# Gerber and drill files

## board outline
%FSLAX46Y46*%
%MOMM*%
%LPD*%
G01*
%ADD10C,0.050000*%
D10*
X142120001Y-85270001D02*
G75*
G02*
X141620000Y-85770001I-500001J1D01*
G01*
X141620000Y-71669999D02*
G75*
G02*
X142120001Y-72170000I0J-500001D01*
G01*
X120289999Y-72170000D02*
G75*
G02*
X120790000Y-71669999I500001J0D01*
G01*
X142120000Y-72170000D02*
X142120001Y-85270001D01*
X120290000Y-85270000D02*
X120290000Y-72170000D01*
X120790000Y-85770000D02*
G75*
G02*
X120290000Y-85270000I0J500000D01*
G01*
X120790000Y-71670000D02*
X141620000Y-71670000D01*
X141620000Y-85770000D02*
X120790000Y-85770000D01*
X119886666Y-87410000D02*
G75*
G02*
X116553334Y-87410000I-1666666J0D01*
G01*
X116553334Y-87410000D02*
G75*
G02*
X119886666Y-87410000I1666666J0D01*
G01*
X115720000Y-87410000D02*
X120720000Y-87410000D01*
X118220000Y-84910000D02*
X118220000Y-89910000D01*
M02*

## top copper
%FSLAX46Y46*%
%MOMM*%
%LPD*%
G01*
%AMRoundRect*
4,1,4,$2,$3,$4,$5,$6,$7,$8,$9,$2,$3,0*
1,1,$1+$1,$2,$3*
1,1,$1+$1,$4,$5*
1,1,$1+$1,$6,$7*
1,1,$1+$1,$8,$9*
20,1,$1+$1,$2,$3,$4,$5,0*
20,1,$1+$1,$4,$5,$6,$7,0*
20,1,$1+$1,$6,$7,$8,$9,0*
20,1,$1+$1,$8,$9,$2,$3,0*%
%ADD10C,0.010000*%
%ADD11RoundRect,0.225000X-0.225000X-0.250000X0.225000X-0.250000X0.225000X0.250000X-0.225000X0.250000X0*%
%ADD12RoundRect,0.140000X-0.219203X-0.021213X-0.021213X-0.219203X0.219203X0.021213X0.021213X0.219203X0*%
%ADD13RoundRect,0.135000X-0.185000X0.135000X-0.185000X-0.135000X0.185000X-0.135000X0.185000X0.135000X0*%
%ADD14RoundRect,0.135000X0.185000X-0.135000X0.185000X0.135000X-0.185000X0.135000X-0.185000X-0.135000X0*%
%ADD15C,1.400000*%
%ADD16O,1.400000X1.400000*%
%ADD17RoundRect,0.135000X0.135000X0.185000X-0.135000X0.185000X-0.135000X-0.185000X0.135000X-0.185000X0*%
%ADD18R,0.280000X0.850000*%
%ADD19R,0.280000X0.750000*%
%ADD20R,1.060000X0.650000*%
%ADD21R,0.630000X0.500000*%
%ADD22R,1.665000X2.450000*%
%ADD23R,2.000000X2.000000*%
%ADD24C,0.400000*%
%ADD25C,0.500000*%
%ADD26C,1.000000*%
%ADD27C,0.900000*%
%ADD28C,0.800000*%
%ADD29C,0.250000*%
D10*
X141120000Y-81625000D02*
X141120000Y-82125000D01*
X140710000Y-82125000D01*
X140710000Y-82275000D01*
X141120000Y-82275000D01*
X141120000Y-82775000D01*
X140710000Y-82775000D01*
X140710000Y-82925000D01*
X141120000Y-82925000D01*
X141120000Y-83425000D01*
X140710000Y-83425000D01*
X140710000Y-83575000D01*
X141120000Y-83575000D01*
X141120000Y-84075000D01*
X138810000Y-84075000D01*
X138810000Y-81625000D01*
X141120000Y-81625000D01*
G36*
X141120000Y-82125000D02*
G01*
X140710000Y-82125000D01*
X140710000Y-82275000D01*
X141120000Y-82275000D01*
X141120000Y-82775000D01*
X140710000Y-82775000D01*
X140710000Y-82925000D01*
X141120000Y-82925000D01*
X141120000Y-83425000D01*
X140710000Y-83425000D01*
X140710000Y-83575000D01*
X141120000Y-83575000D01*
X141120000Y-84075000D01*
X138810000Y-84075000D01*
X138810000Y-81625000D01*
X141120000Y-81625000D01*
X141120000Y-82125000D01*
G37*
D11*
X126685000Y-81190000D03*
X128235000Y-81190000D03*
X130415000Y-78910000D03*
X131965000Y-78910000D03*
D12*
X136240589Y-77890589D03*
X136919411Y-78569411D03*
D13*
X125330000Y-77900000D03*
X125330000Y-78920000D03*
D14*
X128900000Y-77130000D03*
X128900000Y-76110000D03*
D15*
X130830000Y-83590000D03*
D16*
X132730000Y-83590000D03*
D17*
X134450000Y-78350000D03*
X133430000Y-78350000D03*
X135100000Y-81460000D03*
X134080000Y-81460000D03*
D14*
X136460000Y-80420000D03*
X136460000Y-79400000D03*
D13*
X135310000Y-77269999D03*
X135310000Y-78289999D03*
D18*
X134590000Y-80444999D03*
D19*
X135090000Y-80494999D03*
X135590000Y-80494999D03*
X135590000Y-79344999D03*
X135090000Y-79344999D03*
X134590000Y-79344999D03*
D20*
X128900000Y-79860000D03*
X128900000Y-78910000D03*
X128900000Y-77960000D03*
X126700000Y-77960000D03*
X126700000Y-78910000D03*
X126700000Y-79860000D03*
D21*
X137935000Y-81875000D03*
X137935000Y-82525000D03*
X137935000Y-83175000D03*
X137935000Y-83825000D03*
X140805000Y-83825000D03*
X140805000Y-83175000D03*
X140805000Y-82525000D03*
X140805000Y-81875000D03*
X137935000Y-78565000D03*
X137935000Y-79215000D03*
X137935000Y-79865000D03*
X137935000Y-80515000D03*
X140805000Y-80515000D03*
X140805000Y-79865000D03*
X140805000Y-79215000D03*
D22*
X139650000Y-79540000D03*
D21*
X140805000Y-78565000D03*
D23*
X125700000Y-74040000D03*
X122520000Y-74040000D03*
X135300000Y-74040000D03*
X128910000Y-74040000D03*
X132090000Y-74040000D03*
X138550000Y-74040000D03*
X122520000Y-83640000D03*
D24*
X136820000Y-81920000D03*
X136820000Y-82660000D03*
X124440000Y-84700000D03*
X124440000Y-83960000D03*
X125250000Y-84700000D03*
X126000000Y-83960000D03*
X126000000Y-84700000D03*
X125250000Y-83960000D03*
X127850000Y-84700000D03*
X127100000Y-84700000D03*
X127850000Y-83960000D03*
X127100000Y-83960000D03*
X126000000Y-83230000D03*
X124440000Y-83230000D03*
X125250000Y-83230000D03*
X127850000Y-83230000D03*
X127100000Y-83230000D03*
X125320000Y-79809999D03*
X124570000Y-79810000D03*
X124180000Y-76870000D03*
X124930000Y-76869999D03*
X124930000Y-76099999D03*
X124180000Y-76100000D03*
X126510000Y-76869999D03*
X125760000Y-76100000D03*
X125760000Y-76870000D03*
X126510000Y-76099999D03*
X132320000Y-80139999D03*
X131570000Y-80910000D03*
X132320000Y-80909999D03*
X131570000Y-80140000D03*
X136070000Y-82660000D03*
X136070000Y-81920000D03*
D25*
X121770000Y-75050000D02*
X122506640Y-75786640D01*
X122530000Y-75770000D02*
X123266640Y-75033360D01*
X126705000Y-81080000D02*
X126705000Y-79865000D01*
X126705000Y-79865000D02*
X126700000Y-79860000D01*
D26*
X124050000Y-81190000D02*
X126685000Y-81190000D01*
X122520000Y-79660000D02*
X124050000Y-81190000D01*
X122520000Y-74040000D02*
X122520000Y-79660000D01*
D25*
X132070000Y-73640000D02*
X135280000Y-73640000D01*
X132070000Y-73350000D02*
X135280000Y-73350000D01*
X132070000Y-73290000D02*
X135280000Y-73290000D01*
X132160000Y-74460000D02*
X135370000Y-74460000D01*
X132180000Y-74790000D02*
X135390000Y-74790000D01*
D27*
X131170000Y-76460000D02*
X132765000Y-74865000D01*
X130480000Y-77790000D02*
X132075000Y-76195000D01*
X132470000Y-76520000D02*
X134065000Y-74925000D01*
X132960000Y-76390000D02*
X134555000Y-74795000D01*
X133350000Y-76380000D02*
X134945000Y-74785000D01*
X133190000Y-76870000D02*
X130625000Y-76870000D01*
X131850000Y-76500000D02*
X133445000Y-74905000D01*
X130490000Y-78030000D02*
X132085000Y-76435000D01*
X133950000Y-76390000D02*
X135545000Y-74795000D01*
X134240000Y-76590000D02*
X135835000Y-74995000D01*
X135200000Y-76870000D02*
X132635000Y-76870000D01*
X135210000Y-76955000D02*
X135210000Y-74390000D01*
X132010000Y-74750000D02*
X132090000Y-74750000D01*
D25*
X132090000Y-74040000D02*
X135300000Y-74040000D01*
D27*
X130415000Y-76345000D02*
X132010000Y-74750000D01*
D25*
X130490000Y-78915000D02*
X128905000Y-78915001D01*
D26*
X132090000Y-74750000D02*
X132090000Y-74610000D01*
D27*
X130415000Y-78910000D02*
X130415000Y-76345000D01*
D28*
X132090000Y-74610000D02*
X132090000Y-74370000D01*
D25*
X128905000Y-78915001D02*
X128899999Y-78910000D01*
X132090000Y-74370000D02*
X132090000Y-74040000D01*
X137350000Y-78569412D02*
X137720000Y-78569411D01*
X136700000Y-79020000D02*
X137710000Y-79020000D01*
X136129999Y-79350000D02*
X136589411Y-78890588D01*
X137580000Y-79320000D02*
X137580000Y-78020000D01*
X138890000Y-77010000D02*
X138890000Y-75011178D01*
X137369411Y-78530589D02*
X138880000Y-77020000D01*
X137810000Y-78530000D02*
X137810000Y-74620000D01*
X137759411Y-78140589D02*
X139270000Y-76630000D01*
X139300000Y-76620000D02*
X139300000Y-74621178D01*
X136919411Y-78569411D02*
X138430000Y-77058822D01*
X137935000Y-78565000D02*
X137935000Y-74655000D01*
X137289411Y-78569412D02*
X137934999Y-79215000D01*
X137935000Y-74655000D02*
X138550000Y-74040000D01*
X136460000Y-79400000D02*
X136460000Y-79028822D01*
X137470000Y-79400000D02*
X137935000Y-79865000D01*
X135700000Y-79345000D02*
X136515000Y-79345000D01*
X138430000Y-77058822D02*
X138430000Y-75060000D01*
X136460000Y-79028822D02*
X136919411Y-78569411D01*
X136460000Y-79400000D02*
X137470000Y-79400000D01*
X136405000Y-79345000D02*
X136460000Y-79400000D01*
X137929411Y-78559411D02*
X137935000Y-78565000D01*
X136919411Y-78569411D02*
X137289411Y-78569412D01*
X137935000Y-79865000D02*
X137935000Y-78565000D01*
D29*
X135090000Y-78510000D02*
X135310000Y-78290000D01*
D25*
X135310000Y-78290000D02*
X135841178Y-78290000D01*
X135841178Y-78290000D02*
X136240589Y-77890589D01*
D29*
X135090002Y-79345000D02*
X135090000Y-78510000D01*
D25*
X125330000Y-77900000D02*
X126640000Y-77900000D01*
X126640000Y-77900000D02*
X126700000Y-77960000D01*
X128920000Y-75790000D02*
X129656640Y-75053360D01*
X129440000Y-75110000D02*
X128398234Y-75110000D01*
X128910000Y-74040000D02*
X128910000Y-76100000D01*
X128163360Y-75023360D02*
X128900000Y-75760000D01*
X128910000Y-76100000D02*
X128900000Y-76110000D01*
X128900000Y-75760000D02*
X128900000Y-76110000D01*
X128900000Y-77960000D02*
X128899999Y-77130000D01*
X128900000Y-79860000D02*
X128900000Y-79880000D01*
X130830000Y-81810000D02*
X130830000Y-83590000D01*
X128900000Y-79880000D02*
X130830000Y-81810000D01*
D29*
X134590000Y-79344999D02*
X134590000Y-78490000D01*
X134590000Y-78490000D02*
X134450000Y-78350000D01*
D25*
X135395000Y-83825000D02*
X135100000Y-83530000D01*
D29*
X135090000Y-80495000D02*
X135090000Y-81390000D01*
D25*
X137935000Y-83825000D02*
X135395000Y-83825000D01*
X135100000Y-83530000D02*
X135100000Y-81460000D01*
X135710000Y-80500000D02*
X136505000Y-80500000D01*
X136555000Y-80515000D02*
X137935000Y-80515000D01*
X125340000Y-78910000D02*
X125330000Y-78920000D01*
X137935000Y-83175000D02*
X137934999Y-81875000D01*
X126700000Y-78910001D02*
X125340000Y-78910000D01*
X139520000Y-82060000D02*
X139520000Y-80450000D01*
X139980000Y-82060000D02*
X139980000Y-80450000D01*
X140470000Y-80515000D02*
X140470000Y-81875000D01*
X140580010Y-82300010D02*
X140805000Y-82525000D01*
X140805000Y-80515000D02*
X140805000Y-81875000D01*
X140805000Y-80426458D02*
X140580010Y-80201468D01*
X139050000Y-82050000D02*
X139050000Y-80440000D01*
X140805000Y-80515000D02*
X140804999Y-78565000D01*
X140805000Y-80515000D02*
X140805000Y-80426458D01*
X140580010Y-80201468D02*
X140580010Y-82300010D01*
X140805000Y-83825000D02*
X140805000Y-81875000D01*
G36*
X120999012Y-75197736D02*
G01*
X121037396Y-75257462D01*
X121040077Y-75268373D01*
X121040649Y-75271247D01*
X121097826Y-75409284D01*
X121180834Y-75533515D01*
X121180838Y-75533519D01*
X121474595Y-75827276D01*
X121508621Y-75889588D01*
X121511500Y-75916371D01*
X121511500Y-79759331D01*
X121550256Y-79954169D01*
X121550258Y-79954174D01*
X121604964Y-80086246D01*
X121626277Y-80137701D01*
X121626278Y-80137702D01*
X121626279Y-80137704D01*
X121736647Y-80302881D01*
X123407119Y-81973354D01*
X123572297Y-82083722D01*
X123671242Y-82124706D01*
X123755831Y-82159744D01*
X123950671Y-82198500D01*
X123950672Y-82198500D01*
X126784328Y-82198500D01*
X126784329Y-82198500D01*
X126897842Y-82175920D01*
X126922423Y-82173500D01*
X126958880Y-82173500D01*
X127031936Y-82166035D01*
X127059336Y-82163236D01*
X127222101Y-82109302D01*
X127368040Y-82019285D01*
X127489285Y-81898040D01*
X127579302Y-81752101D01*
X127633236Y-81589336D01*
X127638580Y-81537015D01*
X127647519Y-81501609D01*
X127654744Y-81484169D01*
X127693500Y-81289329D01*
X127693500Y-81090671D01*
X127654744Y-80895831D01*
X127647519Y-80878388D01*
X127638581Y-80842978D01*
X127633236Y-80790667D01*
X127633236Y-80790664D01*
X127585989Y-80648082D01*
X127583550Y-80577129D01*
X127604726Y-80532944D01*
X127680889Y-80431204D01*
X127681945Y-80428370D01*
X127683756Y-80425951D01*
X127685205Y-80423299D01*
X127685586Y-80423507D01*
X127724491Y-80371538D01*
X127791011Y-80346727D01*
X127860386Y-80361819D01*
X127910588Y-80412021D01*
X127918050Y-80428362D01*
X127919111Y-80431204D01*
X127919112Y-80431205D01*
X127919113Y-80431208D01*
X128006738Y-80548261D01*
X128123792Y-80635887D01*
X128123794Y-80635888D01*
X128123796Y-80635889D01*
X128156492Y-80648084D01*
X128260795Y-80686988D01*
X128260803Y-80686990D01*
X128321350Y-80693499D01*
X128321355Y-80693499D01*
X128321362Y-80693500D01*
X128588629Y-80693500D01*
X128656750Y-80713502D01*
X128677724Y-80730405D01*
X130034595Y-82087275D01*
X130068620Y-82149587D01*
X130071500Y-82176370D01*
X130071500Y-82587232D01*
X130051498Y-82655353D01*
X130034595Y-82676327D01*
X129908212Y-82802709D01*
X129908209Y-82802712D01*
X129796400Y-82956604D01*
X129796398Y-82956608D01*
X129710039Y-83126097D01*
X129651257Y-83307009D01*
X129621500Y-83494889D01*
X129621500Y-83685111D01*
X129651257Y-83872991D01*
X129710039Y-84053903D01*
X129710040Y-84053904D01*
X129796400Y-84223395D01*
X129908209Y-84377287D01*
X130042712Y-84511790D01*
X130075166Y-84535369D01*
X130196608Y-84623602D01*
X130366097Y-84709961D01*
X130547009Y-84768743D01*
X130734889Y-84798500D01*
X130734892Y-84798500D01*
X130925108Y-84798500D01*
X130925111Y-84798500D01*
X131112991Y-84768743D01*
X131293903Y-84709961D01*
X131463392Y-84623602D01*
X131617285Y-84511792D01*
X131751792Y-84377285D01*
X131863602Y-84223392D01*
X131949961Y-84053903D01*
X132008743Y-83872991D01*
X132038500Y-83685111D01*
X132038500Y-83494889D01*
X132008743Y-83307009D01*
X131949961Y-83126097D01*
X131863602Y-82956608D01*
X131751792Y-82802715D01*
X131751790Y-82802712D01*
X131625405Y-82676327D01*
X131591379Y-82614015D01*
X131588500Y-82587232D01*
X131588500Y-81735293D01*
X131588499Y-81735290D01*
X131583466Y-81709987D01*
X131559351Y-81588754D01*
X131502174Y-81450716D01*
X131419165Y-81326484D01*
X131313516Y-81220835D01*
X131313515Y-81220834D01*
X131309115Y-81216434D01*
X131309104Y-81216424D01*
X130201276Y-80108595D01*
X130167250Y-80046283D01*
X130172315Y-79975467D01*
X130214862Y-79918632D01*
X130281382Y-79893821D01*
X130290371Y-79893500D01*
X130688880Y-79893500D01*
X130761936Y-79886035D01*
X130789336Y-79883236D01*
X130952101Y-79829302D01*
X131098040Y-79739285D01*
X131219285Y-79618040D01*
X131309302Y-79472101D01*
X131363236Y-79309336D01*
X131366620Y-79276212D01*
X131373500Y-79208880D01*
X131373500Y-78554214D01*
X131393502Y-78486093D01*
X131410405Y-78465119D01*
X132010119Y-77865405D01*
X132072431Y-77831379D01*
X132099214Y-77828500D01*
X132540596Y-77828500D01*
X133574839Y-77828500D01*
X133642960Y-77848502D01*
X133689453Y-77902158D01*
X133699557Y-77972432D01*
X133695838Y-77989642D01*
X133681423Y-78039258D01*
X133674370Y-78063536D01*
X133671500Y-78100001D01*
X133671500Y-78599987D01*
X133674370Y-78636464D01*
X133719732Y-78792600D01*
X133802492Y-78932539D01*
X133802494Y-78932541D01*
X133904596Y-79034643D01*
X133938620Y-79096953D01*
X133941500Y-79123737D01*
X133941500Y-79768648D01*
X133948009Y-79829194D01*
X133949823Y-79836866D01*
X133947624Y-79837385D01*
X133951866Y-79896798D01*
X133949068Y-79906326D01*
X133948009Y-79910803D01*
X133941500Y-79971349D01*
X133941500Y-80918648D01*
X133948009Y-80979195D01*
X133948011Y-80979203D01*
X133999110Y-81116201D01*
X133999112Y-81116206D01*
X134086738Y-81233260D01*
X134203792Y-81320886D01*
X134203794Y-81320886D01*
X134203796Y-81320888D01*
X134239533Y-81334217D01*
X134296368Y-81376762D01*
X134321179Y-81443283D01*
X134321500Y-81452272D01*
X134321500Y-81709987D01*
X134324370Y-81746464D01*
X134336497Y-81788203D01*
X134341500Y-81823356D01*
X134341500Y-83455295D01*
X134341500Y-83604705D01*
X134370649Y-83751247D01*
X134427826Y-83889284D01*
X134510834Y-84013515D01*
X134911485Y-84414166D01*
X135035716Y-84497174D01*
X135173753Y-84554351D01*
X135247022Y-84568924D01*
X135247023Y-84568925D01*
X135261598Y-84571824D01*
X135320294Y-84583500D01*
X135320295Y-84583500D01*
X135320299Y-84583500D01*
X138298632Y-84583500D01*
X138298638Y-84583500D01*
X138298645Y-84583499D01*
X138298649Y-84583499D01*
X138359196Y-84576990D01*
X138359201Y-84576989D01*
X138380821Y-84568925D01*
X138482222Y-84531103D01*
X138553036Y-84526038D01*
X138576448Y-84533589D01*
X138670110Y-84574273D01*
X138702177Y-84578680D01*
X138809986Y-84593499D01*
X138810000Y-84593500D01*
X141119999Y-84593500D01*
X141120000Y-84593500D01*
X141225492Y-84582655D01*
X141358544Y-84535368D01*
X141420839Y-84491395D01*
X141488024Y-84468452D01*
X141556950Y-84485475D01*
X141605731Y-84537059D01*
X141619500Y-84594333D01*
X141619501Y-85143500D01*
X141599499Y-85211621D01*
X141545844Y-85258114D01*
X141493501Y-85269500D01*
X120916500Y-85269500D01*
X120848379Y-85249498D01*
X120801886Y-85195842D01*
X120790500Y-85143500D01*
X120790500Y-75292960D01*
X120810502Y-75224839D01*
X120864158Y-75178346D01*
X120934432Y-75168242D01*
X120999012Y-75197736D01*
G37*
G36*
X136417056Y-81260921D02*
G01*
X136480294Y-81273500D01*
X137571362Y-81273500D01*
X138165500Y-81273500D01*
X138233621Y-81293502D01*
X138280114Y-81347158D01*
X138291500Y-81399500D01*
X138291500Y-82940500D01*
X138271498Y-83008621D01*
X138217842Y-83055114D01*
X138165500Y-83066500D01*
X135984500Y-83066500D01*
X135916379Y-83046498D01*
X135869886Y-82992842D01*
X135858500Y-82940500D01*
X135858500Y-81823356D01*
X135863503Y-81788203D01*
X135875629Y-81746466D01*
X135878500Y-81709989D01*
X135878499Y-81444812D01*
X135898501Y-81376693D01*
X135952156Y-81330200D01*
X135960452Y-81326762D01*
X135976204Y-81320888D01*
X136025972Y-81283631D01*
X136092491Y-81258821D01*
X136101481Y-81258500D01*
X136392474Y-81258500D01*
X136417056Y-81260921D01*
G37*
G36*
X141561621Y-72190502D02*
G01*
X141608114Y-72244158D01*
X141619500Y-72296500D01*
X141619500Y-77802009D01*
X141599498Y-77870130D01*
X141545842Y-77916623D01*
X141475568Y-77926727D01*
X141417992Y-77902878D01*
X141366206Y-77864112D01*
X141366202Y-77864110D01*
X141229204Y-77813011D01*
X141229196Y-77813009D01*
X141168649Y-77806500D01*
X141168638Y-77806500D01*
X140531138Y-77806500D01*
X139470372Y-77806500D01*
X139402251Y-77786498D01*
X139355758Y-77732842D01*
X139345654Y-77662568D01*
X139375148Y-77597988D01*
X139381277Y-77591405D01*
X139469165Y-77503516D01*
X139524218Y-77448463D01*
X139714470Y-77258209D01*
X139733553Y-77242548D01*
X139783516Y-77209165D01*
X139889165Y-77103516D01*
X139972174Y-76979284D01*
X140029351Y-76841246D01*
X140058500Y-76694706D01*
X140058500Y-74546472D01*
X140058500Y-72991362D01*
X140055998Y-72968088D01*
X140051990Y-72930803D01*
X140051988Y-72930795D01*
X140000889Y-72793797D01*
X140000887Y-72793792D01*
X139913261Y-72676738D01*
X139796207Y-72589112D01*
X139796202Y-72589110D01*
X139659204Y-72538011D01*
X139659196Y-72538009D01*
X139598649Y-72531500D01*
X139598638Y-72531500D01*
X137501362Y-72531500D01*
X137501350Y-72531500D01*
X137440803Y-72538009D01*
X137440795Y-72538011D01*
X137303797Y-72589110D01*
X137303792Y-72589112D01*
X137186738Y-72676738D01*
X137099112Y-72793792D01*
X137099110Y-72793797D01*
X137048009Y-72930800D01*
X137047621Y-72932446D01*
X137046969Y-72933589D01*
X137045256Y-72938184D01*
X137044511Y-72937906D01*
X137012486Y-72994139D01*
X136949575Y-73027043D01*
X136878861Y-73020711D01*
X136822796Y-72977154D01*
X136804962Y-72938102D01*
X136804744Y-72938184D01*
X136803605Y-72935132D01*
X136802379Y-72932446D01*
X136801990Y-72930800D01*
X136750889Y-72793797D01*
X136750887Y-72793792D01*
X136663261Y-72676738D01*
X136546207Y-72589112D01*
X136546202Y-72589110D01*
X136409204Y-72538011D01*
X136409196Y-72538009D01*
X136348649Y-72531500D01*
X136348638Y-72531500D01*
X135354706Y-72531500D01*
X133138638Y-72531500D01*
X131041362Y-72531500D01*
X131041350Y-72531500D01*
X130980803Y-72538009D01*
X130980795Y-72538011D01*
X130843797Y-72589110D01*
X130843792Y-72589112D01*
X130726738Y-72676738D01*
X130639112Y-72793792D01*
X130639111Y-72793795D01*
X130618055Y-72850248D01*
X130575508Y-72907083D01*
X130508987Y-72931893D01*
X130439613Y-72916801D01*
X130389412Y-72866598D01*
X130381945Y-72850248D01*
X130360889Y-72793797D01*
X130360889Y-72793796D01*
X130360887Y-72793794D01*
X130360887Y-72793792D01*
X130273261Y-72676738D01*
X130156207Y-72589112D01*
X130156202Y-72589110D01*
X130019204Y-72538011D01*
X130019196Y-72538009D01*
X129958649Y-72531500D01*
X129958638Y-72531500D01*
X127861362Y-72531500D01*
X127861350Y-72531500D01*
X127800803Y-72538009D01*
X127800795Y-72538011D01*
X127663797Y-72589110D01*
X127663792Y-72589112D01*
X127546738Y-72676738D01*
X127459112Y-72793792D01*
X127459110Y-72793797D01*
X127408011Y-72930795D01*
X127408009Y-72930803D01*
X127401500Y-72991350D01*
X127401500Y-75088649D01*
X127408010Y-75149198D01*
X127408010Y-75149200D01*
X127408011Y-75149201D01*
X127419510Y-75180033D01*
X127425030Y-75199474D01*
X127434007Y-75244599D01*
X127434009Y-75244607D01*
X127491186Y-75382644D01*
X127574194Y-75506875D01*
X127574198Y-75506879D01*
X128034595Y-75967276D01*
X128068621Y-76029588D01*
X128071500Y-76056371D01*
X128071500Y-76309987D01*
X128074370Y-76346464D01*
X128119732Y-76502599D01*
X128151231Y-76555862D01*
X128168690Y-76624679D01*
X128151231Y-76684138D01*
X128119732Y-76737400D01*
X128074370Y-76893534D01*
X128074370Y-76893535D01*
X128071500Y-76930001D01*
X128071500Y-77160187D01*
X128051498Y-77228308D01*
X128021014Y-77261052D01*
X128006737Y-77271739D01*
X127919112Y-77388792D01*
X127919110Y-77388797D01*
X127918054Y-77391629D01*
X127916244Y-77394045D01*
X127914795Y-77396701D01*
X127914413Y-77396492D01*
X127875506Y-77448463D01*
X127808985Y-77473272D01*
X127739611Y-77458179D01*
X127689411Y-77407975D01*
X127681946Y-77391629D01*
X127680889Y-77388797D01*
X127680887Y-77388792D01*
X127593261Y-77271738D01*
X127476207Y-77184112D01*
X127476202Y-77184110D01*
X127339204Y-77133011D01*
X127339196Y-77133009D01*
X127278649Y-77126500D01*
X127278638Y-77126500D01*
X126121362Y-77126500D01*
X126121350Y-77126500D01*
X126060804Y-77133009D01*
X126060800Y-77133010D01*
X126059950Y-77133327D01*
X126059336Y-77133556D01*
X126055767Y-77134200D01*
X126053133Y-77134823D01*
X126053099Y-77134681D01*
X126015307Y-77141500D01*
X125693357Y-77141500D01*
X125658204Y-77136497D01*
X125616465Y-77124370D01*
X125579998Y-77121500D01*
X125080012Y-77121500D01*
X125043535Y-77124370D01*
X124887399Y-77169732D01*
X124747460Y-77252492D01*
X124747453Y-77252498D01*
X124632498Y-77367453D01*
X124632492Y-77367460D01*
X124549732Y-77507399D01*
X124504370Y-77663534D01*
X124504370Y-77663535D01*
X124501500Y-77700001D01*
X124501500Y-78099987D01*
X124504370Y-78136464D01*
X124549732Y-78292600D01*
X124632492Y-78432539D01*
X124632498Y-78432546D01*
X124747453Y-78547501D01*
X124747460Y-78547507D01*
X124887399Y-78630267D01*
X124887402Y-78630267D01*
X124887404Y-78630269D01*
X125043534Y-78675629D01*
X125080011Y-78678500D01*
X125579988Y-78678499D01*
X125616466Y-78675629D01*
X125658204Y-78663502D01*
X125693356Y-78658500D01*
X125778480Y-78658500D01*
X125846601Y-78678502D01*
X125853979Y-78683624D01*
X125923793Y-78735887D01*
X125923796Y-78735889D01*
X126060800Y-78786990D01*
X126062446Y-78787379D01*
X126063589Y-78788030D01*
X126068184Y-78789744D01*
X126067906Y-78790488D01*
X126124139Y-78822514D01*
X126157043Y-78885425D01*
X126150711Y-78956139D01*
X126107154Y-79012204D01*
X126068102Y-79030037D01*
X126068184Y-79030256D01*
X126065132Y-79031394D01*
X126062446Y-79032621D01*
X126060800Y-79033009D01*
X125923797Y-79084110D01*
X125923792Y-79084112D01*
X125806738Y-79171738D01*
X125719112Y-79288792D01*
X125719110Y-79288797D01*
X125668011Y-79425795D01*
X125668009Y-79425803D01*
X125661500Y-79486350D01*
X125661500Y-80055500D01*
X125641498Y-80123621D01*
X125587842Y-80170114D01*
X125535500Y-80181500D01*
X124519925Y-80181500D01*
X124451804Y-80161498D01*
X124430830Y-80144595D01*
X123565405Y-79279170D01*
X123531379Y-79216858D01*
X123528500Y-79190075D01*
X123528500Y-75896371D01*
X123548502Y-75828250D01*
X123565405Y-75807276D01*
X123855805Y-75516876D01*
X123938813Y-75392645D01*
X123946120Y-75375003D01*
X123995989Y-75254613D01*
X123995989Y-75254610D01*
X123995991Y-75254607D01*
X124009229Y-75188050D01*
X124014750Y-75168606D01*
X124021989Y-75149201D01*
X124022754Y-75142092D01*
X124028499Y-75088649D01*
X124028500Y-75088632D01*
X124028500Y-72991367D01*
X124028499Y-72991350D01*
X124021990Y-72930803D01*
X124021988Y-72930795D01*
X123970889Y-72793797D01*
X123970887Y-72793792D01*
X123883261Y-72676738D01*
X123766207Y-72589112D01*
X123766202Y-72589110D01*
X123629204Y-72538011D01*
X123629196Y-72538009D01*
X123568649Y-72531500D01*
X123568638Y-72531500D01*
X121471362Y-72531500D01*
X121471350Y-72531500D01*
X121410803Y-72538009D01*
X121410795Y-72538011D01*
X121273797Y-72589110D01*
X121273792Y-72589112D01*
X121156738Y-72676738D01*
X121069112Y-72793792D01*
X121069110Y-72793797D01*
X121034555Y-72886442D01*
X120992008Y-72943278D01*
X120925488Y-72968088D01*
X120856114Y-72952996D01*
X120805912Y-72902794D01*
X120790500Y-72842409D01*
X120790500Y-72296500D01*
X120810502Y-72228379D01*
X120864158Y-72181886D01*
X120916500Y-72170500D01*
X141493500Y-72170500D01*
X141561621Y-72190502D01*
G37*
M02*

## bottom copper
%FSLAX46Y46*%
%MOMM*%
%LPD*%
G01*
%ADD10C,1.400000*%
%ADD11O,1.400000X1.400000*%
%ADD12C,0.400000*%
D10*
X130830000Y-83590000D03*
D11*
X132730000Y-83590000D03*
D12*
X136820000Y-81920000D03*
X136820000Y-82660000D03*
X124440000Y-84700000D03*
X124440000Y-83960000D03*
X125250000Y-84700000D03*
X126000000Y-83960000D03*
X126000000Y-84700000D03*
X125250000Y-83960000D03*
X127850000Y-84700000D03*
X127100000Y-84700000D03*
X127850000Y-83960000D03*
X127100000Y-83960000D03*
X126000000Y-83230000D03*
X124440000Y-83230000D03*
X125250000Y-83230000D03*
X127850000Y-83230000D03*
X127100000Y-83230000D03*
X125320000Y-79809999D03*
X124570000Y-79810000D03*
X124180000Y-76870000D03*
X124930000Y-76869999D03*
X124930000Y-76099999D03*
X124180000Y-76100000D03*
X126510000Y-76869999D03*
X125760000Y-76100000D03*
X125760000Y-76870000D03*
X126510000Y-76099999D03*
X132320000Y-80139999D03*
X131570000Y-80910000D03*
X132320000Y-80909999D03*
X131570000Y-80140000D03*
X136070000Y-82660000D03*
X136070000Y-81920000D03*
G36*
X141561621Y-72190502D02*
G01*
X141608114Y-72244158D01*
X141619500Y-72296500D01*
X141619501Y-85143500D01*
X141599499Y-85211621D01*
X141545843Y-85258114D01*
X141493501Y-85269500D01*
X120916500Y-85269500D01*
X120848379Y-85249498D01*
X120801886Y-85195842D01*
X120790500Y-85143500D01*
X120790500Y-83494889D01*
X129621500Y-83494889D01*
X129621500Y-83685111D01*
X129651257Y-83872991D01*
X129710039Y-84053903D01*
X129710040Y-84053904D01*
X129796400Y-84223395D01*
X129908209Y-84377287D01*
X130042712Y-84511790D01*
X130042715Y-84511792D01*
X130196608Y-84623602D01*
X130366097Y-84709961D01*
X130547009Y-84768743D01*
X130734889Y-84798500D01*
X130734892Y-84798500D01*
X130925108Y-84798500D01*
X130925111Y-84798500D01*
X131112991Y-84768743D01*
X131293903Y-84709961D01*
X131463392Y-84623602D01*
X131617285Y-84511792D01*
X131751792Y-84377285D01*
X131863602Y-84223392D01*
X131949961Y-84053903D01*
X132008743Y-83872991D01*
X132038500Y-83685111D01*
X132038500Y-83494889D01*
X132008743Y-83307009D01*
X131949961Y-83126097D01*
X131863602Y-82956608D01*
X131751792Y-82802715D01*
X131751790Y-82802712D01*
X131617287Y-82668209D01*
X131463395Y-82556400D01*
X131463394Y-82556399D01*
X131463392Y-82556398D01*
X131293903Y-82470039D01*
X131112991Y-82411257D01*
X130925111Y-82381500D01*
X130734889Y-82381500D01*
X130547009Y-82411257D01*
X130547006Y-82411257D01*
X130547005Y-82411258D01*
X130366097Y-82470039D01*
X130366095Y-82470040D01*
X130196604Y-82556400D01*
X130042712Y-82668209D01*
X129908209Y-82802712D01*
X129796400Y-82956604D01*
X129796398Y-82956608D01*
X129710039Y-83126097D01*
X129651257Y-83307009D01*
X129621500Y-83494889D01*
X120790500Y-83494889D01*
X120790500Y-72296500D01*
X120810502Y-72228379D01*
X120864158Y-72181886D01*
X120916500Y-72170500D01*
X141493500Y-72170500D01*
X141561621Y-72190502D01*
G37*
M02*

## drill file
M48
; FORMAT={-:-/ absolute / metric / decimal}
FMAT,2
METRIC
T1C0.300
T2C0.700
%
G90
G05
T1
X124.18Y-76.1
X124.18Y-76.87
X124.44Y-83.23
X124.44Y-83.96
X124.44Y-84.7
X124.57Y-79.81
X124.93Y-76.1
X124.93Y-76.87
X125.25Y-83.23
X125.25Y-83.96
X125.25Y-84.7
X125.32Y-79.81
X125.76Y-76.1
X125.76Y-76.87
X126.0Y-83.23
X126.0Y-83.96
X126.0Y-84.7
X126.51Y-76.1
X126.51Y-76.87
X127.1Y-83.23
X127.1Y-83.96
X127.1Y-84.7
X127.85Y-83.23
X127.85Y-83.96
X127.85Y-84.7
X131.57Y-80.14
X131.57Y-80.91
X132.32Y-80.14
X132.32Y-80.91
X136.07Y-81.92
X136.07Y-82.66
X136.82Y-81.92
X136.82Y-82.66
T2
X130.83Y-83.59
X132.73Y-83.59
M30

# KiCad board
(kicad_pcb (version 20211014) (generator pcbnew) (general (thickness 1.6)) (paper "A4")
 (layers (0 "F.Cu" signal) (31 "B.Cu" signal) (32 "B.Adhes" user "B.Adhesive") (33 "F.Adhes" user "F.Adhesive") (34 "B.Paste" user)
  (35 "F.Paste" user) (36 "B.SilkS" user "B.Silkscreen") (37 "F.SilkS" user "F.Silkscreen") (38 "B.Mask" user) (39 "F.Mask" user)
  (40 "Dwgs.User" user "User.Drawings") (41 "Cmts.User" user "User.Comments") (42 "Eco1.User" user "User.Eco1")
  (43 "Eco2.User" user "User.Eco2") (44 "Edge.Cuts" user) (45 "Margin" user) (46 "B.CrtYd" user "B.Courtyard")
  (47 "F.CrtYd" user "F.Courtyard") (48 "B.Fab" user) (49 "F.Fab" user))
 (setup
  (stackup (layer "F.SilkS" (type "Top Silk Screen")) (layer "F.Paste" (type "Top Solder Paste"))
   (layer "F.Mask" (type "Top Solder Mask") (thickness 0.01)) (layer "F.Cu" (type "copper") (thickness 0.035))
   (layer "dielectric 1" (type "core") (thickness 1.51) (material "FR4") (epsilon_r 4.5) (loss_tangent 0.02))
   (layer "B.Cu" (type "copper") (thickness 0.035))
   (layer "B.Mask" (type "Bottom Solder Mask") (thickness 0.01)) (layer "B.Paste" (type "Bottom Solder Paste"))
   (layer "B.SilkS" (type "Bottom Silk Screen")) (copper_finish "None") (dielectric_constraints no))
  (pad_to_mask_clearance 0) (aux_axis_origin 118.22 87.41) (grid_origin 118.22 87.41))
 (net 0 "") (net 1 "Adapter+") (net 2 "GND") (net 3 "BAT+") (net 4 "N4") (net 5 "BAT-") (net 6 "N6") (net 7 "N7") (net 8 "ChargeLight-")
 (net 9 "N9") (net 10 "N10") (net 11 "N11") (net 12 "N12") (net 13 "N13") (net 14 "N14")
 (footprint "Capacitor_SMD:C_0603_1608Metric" (layer "F.Cu") (at 127.46 81.19)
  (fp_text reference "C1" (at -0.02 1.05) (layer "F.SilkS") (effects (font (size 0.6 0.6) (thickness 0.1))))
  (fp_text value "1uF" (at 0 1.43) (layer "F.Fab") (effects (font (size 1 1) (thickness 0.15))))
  (pad "1" smd roundrect locked (at -0.775 0) (size 0.9 0.95) (layers "F.Cu" "F.Paste" "F.Mask") (roundrect_rratio 0.25) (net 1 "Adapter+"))
  (pad "2" smd roundrect locked (at 0.775 0) (size 0.9 0.95) (layers "F.Cu" "F.Paste" "F.Mask") (roundrect_rratio 0.25) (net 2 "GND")))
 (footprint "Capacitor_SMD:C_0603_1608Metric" (layer "F.Cu") (at 131.19 78.91)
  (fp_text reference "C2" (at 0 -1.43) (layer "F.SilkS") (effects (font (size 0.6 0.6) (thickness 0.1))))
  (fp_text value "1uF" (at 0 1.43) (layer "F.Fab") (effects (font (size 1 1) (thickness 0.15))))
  (pad "1" smd roundrect locked (at -0.775 0) (size 0.9 0.95) (layers "F.Cu" "F.Paste" "F.Mask") (roundrect_rratio 0.25) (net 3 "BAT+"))
  (pad "2" smd roundrect locked (at 0.775 0) (size 0.9 0.95) (layers "F.Cu" "F.Paste" "F.Mask") (roundrect_rratio 0.25) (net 2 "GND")))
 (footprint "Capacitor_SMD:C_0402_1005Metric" (layer "F.Cu") (at 136.58 78.23 -45)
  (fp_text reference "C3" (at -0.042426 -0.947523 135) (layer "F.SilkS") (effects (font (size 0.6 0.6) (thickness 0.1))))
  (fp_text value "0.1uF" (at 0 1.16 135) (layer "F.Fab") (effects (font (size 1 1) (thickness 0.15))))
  (pad "1" smd roundrect locked (at -0.48 0 315) (size 0.56 0.62) (layers "F.Cu" "F.Paste" "F.Mask") (roundrect_rratio 0.25) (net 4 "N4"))
  (pad "2" smd roundrect locked (at 0.48 0 315) (size 0.56 0.62) (layers "F.Cu" "F.Paste" "F.Mask") (roundrect_rratio 0.25) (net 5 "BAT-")))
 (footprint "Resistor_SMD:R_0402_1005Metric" (layer "F.Cu") (at 125.33 78.41 -90)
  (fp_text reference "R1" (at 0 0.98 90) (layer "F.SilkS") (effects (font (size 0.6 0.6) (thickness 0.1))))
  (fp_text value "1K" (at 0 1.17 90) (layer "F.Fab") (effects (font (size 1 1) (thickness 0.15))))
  (pad "1" smd roundrect locked (at -0.51 0 270) (size 0.54 0.64) (layers "F.Cu" "F.Paste" "F.Mask") (roundrect_rratio 0.25) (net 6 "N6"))
  (pad "2" smd roundrect locked (at 0.51 0 270) (size 0.54 0.64) (layers "F.Cu" "F.Paste" "F.Mask") (roundrect_rratio 0.25) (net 2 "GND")))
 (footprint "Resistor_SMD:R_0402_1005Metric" (layer "F.Cu") (at 128.9 76.62 90)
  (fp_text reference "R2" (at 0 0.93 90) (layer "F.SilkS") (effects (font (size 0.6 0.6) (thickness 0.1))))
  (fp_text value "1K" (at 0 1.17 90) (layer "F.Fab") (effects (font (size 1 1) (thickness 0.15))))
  (pad "1" smd roundrect locked (at -0.51 0 90) (size 0.54 0.64) (layers "F.Cu" "F.Paste" "F.Mask") (roundrect_rratio 0.25) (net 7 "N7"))
  (pad "2" smd roundrect locked (at 0.51 0 90) (size 0.54 0.64) (layers "F.Cu" "F.Paste" "F.Mask") (roundrect_rratio 0.25)
   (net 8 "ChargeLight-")))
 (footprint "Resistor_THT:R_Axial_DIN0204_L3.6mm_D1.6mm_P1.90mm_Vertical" (layer "F.Cu") (at 130.83 83.59)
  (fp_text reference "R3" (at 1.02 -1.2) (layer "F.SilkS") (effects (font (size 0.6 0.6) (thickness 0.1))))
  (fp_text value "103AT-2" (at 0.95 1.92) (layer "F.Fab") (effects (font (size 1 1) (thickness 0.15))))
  (pad "1" thru_hole circle locked (at 0 0) (size 1.4 1.4) (drill 0.7) (layers *.Cu *.Mask) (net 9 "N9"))
  (pad "2" thru_hole oval locked (at 1.9 0) (size 1.4 1.4) (drill 0.7) (layers *.Cu *.Mask) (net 2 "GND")))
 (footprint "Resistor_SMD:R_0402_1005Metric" (layer "F.Cu") (at 133.94 78.35 180)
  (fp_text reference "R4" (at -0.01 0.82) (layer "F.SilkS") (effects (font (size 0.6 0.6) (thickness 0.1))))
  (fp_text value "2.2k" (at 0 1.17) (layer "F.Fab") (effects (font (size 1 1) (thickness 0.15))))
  (pad "1" smd roundrect locked (at -0.51 0 180) (size 0.54 0.64) (layers "F.Cu" "F.Paste" "F.Mask") (roundrect_rratio 0.25) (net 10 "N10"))
  (pad "2" smd roundrect locked (at 0.51 0 180) (size 0.54 0.64) (layers "F.Cu" "F.Paste" "F.Mask") (roundrect_rratio 0.25) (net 2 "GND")))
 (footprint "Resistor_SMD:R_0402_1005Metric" (layer "F.Cu") (at 134.59 81.46 180)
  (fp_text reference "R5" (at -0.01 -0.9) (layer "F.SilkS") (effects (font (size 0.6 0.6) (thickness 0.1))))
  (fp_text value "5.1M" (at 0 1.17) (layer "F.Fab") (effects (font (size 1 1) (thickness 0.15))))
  (pad "1" smd roundrect locked (at -0.51 0 180) (size 0.54 0.64) (layers "F.Cu" "F.Paste" "F.Mask") (roundrect_rratio 0.25) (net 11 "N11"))
  (pad "2" smd roundrect locked (at 0.51 0 180) (size 0.54 0.64) (layers "F.Cu" "F.Paste" "F.Mask") (roundrect_rratio 0.25) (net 2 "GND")))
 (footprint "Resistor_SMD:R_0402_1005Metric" (layer "F.Cu") (at 136.46 79.91 90)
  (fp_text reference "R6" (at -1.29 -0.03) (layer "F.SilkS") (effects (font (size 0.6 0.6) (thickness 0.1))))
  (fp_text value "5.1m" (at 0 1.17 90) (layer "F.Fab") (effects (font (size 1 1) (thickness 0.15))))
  (pad "1" smd roundrect locked (at -0.51 0 90) (size 0.54 0.64) (layers "F.Cu" "F.Paste" "F.Mask") (roundrect_rratio 0.25) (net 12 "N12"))
  (pad "2" smd roundrect locked (at 0.51 0 90) (size 0.54 0.64) (layers "F.Cu" "F.Paste" "F.Mask") (roundrect_rratio 0.25) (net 5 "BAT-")))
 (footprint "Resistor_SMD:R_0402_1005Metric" (layer "F.Cu") (at 135.31 77.779999 -90)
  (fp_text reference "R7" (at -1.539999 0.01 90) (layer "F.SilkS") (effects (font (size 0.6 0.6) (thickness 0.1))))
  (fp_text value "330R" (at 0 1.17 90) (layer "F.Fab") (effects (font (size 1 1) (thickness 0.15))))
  (pad "1" smd roundrect locked (at -0.51 0 270) (size 0.54 0.64) (layers "F.Cu" "F.Paste" "F.Mask") (roundrect_rratio 0.25) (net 3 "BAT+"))
  (pad "2" smd roundrect locked (at 0.51 0 270) (size 0.54 0.64) (layers "F.Cu" "F.Paste" "F.Mask") (roundrect_rratio 0.25) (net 4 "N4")))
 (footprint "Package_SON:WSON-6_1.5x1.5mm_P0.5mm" (layer "F.Cu") (at 135.09 79.919999 90)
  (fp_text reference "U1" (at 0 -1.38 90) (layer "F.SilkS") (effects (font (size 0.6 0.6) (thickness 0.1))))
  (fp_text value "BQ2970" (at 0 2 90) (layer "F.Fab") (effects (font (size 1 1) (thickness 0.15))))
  (pad "1" smd rect locked (at -0.525 -0.5) (size 0.28 0.85) (layers "F.Cu" "F.Paste" "F.Mask") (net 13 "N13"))
  (pad "2" smd rect locked (at -0.575 0) (size 0.28 0.75) (layers "F.Cu" "F.Paste" "F.Mask") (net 11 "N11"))
  (pad "3" smd rect locked (at -0.575 0.5) (size 0.28 0.75) (layers "F.Cu" "F.Paste" "F.Mask") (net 12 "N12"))
  (pad "4" smd rect locked (at 0.575 0.5) (size 0.28 0.75) (layers "F.Cu" "F.Paste" "F.Mask") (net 5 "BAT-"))
  (pad "5" smd rect locked (at 0.575 0) (size 0.28 0.75) (layers "F.Cu" "F.Paste" "F.Mask") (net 4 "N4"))
  (pad "6" smd rect locked (at 0.575 -0.5) (size 0.28 0.75) (layers "F.Cu" "F.Paste" "F.Mask") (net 10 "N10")))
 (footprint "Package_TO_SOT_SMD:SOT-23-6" (layer "F.Cu") (at 127.8 78.91 180)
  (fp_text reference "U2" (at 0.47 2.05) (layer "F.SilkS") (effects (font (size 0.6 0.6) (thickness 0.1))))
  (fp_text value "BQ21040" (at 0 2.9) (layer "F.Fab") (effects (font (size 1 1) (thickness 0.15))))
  (pad "1" smd rect locked (at -1.1 -0.95 180) (size 1.06 0.65) (layers "F.Cu" "F.Paste" "F.Mask") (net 9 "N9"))
  (pad "2" smd rect locked (at -1.1 0 180) (size 1.06 0.65) (layers "F.Cu" "F.Paste" "F.Mask") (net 3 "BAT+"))
  (pad "3" smd rect locked (at -1.1 0.95 180) (size 1.06 0.65) (layers "F.Cu" "F.Paste" "F.Mask") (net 7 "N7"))
  (pad "4" smd rect locked (at 1.1 0.95 180) (size 1.06 0.65) (layers "F.Cu" "F.Paste" "F.Mask") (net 6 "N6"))
  (pad "5" smd rect locked (at 1.1 0 180) (size 1.06 0.65) (layers "F.Cu" "F.Paste" "F.Mask") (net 2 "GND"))
  (pad "6" smd rect locked (at 1.1 -0.95 180) (size 1.06 0.65) (layers "F.Cu" "F.Paste" "F.Mask") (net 1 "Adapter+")))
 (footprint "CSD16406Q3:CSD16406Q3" (layer "F.Cu") (at 139.37 82.85)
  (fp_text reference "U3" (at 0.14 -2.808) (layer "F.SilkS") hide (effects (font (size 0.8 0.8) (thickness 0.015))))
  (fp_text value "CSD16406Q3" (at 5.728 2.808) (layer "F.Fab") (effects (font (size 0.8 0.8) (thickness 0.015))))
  (fp_poly
   (pts (xy 1.75 -1.225) (xy 1.75 -0.725) (xy 1.34 -0.725) (xy 1.34 -0.575) (xy 1.75 -0.575) (xy 1.75 -0.075) (xy 1.34 -0.075)
    (xy 1.34 0.075) (xy 1.75 0.075) (xy 1.75 0.575) (xy 1.34 0.575) (xy 1.34 0.725) (xy 1.75 0.725) (xy 1.75 1.225) (xy -0.56 1.225)
    (xy -0.56 -1.225))
   (layer "F.Cu") (width 0.01) (fill solid))
  (pad "1" smd rect locked (at -1.435 -0.975) (size 0.63 0.5) (layers "F.Cu" "F.Mask") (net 2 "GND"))
  (pad "2" smd rect locked (at -1.435 -0.325) (size 0.63 0.5) (layers "F.Cu" "F.Mask") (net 2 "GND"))
  (pad "3" smd rect locked (at -1.435 0.325) (size 0.63 0.5) (layers "F.Cu" "F.Mask") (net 2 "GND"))
  (pad "4" smd rect locked (at -1.435 0.975) (size 0.63 0.5) (layers "F.Cu" "F.Mask") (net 11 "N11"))
  (pad "5" smd rect locked (at 1.435 0.975) (size 0.63 0.5) (layers "F.Cu") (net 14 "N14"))
  (pad "6" smd rect locked (at 1.435 0.325) (size 0.63 0.5) (layers "F.Cu") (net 14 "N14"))
  (pad "7" smd rect locked (at 1.435 -0.325) (size 0.63 0.5) (layers "F.Cu") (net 14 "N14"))
  (pad "8" smd rect locked (at 1.435 -0.975) (size 0.63 0.5) (layers "F.Cu") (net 14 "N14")))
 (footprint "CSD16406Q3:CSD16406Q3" (layer "F.Cu") (at 139.37 79.54)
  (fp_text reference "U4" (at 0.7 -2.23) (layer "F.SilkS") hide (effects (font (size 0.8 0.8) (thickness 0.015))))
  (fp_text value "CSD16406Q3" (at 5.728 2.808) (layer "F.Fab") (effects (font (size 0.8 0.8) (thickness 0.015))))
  (pad "1" smd rect (at -1.435 -0.975) (size 0.63 0.5) (layers "F.Cu" "F.Mask") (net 5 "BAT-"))
  (pad "2" smd rect (at -1.435 -0.325) (size 0.63 0.5) (layers "F.Cu" "F.Mask") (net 5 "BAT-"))
  (pad "3" smd rect (at -1.435 0.325) (size 0.63 0.5) (layers "F.Cu" "F.Mask") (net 5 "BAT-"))
  (pad "4" smd rect (at -1.435 0.975) (size 0.63 0.5) (layers "F.Cu" "F.Mask") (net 12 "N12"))
  (pad "5" smd rect (at 1.435 0.975) (size 0.63 0.5) (layers "F.Cu") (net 14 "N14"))
  (pad "6" smd rect (at 1.435 0.325) (size 0.63 0.5) (layers "F.Cu") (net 14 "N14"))
  (pad "7" smd rect (at 1.435 -0.325) (size 0.63 0.5) (layers "F.Cu") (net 14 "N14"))
  (pad "8" smd rect (at 0.28 0) (size 1.665 2.45) (layers "F.Cu") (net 14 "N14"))
  (pad "8" smd rect (at 1.435 -0.975) (size 0.63 0.5) (layers "F.Cu") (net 14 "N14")))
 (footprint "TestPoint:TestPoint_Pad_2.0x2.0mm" (layer "F.Cu") (at 125.7 74.04 180)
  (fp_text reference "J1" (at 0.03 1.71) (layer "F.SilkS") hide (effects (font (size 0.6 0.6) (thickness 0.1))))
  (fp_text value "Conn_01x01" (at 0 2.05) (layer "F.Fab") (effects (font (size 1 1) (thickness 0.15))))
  (pad "1" smd rect locked (at 0 0 180) (size 2 2) (layers "F.Cu" "F.Mask") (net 2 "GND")))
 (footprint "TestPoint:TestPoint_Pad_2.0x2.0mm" (layer "F.Cu") (at 122.52 74.04 180)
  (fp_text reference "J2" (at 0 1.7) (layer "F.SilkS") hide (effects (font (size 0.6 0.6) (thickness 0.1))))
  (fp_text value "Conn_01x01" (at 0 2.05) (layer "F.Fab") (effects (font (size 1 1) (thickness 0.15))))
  (pad "1" smd rect locked (at 0 0 180) (size 2 2) (layers "F.Cu" "F.Mask") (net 1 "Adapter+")))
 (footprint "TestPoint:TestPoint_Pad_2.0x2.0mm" (layer "F.Cu") (at 135.3 74.04 180)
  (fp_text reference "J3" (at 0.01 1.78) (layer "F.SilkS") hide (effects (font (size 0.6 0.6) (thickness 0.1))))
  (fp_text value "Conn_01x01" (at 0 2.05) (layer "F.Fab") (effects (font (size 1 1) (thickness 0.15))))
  (pad "1" smd rect locked (at 0 0 180) (size 2 2) (layers "F.Cu" "F.Mask") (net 3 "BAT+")))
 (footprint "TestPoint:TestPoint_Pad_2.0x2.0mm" (layer "F.Cu") (at 128.91 74.04 180)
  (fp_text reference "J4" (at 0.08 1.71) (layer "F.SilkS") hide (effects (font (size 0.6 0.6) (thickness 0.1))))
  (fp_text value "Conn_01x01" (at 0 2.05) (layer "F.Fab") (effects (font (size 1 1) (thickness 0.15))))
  (pad "1" smd rect locked (at 0 0 180) (size 2 2) (layers "F.Cu" "F.Mask") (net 8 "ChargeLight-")))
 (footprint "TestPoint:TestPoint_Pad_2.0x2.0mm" (layer "F.Cu") (at 132.09 74.04 180)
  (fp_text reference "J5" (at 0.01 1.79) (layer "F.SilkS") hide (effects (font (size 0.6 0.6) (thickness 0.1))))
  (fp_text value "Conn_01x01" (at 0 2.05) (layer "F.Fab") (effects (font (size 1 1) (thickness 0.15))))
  (pad "1" smd rect locked (at 0 0 180) (size 2 2) (layers "F.Cu" "F.Mask") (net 3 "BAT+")))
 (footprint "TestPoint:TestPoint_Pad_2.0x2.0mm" (layer "F.Cu") (at 138.55 74.04 180)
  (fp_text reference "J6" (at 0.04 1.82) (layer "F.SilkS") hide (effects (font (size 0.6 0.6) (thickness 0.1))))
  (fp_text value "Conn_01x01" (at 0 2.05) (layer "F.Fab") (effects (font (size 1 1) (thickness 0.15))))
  (pad "1" smd rect locked (at 0 0 180) (size 2 2) (layers "F.Cu" "F.Mask") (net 5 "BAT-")))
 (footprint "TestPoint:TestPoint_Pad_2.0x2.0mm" (layer "F.Cu") (at 122.52 83.64)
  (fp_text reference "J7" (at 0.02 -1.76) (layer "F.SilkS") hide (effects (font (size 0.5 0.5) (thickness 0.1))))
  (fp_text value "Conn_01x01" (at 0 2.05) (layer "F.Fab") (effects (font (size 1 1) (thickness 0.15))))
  (pad "1" smd rect locked (at 0 0) (size 2 2) (layers "F.Cu" "F.Mask") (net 2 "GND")))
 (gr_arc (start 142.120001 85.270001) (mid 141.973554 85.623554) (end 141.62 85.77) (layer "Edge.Cuts") (width 0.05))
 (gr_arc (start 141.62 71.669999) (mid 141.973553 71.816446) (end 142.12 72.17) (layer "Edge.Cuts") (width 0.05))
 (gr_arc (start 120.289999 72.17) (mid 120.436446 71.816447) (end 120.79 71.67) (layer "Edge.Cuts") (width 0.05))
 (gr_line (start 142.12 72.17) (end 142.120001 85.270001) (layer "Edge.Cuts") (width 0.05))
 (gr_line (start 120.29 85.27) (end 120.29 72.17) (layer "Edge.Cuts") (width 0.05))
 (gr_arc (start 120.79 85.77) (mid 120.436447 85.623553) (end 120.29 85.27) (layer "Edge.Cuts") (width 0.05))
 (gr_line (start 120.79 71.67) (end 141.62 71.67) (layer "Edge.Cuts") (width 0.05))
 (gr_line (start 141.62 85.77) (end 120.79 85.77) (layer "Edge.Cuts") (width 0.05))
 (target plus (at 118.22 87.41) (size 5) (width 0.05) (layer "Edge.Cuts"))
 (segment (start 121.77 75.05) (end 122.50664 75.78664) (width 0.5) (layer "F.Cu") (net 1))
 (segment (start 122.53 75.77) (end 123.26664 75.03336) (width 0.5) (layer "F.Cu") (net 1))
 (segment (start 126.705 81.08) (end 126.705 79.865) (width 0.5) (layer "F.Cu") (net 1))
 (segment (start 126.705 79.865) (end 126.7 79.86) (width 0.5) (layer "F.Cu") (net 1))
 (segment (start 124.05 81.19) (end 126.685 81.19) (width 1) (layer "F.Cu") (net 1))
 (segment (start 122.52 79.66) (end 124.05 81.19) (width 1) (layer "F.Cu") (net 1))
 (segment (start 122.52 74.04) (end 122.52 79.66) (width 1) (layer "F.Cu") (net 1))
 (segment (start 132.07 73.64) (end 135.28 73.64) (width 0.5) (layer "F.Cu") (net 3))
 (segment (start 132.07 73.35) (end 135.28 73.35) (width 0.5) (layer "F.Cu") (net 3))
 (segment (start 132.07 73.29) (end 135.28 73.29) (width 0.5) (layer "F.Cu") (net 3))
 (segment (start 132.16 74.46) (end 135.37 74.46) (width 0.5) (layer "F.Cu") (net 3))
 (segment (start 132.18 74.79) (end 135.39 74.79) (width 0.5) (layer "F.Cu") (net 3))
 (segment (start 131.17 76.46) (end 132.765 74.865) (width 0.9) (layer "F.Cu") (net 3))
 (segment (start 130.48 77.79) (end 132.075 76.195) (width 0.9) (layer "F.Cu") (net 3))
 (segment (start 132.47 76.52) (end 134.065 74.925) (width 0.9) (layer "F.Cu") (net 3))
 (segment (start 132.96 76.39) (end 134.555 74.795) (width 0.9) (layer "F.Cu") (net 3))
 (segment (start 133.35 76.38) (end 134.945 74.785) (width 0.9) (layer "F.Cu") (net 3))
 (segment (start 133.19 76.87) (end 130.625 76.87) (width 0.9) (layer "F.Cu") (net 3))
 (segment (start 131.85 76.5) (end 133.445 74.905) (width 0.9) (layer "F.Cu") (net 3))
 (segment (start 130.49 78.03) (end 132.085 76.435) (width 0.9) (layer "F.Cu") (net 3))
 (segment (start 133.95 76.39) (end 135.545 74.795) (width 0.9) (layer "F.Cu") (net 3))
 (segment (start 134.24 76.59) (end 135.835 74.995) (width 0.9) (layer "F.Cu") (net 3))
 (segment (start 135.2 76.87) (end 132.635 76.87) (width 0.9) (layer "F.Cu") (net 3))
 (segment (start 135.21 76.955) (end 135.21 74.39) (width 0.9) (layer "F.Cu") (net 3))
 (segment (start 132.01 74.75) (end 132.09 74.75) (width 0.9) (layer "F.Cu") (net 3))
 (segment (start 132.09 74.04) (end 135.3 74.04) (width 0.5) (layer "F.Cu") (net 3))
 (segment (start 130.415 76.345) (end 132.01 74.75) (width 0.9) (layer "F.Cu") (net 3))
 (segment (start 130.49 78.915) (end 128.905 78.915001) (width 0.5) (layer "F.Cu") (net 3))
 (segment (start 132.09 74.75) (end 132.09 74.61) (width 1) (layer "F.Cu") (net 3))
 (segment (start 130.415 78.91) (end 130.415 76.345) (width 0.9) (layer "F.Cu") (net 3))
 (segment (start 132.09 74.61) (end 132.09 74.37) (width 0.8) (layer "F.Cu") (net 3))
 (segment (start 128.905 78.915001) (end 128.899999 78.91) (width 0.5) (layer "F.Cu") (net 3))
 (segment (start 132.09 74.37) (end 132.09 74.04) (width 0.5) (layer "F.Cu") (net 3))
 (segment (start 137.35 78.569412) (end 137.72 78.569411) (width 0.5) (layer "F.Cu") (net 5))
 (segment (start 136.7 79.02) (end 137.71 79.02) (width 0.5) (layer "F.Cu") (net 5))
 (segment (start 136.129999 79.35) (end 136.589411 78.890588) (width 0.5) (layer "F.Cu") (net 5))
 (segment (start 137.58 79.32) (end 137.58 78.02) (width 0.5) (layer "F.Cu") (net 5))
 (segment (start 138.89 77.01) (end 138.89 75.011178) (width 0.5) (layer "F.Cu") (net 5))
 (segment (start 137.369411 78.530589) (end 138.88 77.02) (width 0.5) (layer "F.Cu") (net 5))
 (segment (start 137.81 78.53) (end 137.81 74.62) (width 0.5) (layer "F.Cu") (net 5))
 (segment (start 137.759411 78.140589) (end 139.27 76.63) (width 0.5) (layer "F.Cu") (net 5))
 (segment (start 139.3 76.62) (end 139.3 74.621178) (width 0.5) (layer "F.Cu") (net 5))
 (segment (start 136.919411 78.569411) (end 138.43 77.058822) (width 0.5) (layer "F.Cu") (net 5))
 (segment (start 137.935 78.565) (end 137.935 74.655) (width 0.5) (layer "F.Cu") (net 5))
 (segment (start 137.289411 78.569412) (end 137.934999 79.215) (width 0.5) (layer "F.Cu") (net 5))
 (segment (start 137.935 74.655) (end 138.55 74.04) (width 0.5) (layer "F.Cu") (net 5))
 (segment (start 136.46 79.4) (end 136.46 79.028822) (width 0.5) (layer "F.Cu") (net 5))
 (segment (start 137.47 79.4) (end 137.935 79.865) (width 0.5) (layer "F.Cu") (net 5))
 (segment (start 135.7 79.345) (end 136.515 79.345) (width 0.5) (layer "F.Cu") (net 5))
 (segment (start 138.43 77.058822) (end 138.43 75.06) (width 0.5) (layer "F.Cu") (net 5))
 (segment (start 136.46 79.028822) (end 136.919411 78.569411) (width 0.5) (layer "F.Cu") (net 5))
 (segment (start 136.46 79.4) (end 137.47 79.4) (width 0.5) (layer "F.Cu") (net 5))
 (segment (start 136.405 79.345) (end 136.46 79.4) (width 0.5) (layer "F.Cu") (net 5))
 (segment (start 137.929411 78.559411) (end 137.935 78.565) (width 0.5) (layer "F.Cu") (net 5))
 (segment (start 136.919411 78.569411) (end 137.289411 78.569412) (width 0.5) (layer "F.Cu") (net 5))
 (segment (start 137.935 79.865) (end 137.935 78.565) (width 0.5) (layer "F.Cu") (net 5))
 (segment (start 135.09 78.51) (end 135.31 78.29) (width 0.25) (layer "F.Cu") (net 4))
 (segment (start 135.31 78.29) (end 135.841178 78.29) (width 0.5) (layer "F.Cu") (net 4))
 (segment (start 135.841178 78.29) (end 136.240589 77.890589) (width 0.5) (layer "F.Cu") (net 4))
 (segment (start 135.090002 79.345) (end 135.09 78.51) (width 0.25) (layer "F.Cu") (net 4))
 (segment (start 125.33 77.9) (end 126.64 77.9) (width 0.5) (layer "F.Cu") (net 6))
 (segment (start 126.64 77.9) (end 126.7 77.96) (width 0.5) (layer "F.Cu") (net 6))
 (segment (start 128.92 75.79) (end 129.65664 75.05336) (width 0.5) (layer "F.Cu") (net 8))
 (segment (start 129.44 75.11) (end 128.398234 75.11) (width 0.5) (layer "F.Cu") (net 8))
 (segment (start 128.91 74.04) (end 128.91 76.1) (width 0.5) (layer "F.Cu") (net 8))
 (segment (start 128.16336 75.02336) (end 128.9 75.76) (width 0.5) (layer "F.Cu") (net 8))
 (segment (start 128.91 76.1) (end 128.9 76.11) (width 0.5) (layer "F.Cu") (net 8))
 (segment (start 128.9 75.76) (end 128.9 76.11) (width 0.5) (layer "F.Cu") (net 8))
 (segment (start 128.9 77.96) (end 128.899999 77.13) (width 0.5) (layer "F.Cu") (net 7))
 (segment (start 128.9 79.86) (end 128.9 79.88) (width 0.5) (layer "F.Cu") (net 9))
 (segment (start 130.83 81.81) (end 130.83 83.59) (width 0.5) (layer "F.Cu") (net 9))
 (segment (start 128.9 79.88) (end 130.83 81.81) (width 0.5) (layer "F.Cu") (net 9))
 (segment (start 134.59 79.344999) (end 134.59 78.49) (width 0.25) (layer "F.Cu") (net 10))
 (segment (start 134.59 78.49) (end 134.45 78.35) (width 0.25) (layer "F.Cu") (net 10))
 (segment (start 135.395 83.825) (end 135.1 83.53) (width 0.5) (layer "F.Cu") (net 11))
 (segment (start 135.09 80.495) (end 135.09 81.39) (width 0.25) (layer "F.Cu") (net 11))
 (segment (start 137.935 83.825) (end 135.395 83.825) (width 0.5) (layer "F.Cu") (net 11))
 (segment (start 135.1 83.53) (end 135.1 81.46) (width 0.5) (layer "F.Cu") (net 11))
 (segment (start 135.71 80.5) (end 136.505 80.5) (width 0.5) (layer "F.Cu") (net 12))
 (segment (start 136.555 80.515) (end 137.935 80.515) (width 0.5) (layer "F.Cu") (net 12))
 (segment (start 125.34 78.91) (end 125.33 78.92) (width 0.5) (layer "F.Cu") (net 2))
 (segment (start 137.935 83.175) (end 137.934999 81.875) (width 0.5) (layer "F.Cu") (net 2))
 (segment (start 126.7 78.910001) (end 125.34 78.91) (width 0.5) (layer "F.Cu") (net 2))
 (via (at 136.82 81.92) (size 0.4) (drill 0.3) (layers "F.Cu" "B.Cu") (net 2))
 (via (at 136.82 82.66) (size 0.4) (drill 0.3) (layers "F.Cu" "B.Cu") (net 2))
 (via (at 124.44 84.7) (size 0.4) (drill 0.3) (layers "F.Cu" "B.Cu") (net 2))
 (via (at 124.44 83.96) (size 0.4) (drill 0.3) (layers "F.Cu" "B.Cu") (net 2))
 (via (at 125.25 84.7) (size 0.4) (drill 0.3) (layers "F.Cu" "B.Cu") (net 2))
 (via (at 126 83.96) (size 0.4) (drill 0.3) (layers "F.Cu" "B.Cu") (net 2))
 (via (at 126 84.7) (size 0.4) (drill 0.3) (layers "F.Cu" "B.Cu") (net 2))
 (via (at 125.25 83.96) (size 0.4) (drill 0.3) (layers "F.Cu" "B.Cu") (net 2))
 (via (at 127.85 84.7) (size 0.4) (drill 0.3) (layers "F.Cu" "B.Cu") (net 2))
 (via (at 127.1 84.7) (size 0.4) (drill 0.3) (layers "F.Cu" "B.Cu") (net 2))
 (via (at 127.85 83.96) (size 0.4) (drill 0.3) (layers "F.Cu" "B.Cu") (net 2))
 (via (at 127.1 83.96) (size 0.4) (drill 0.3) (layers "F.Cu" "B.Cu") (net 2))
 (via (at 126 83.23) (size 0.4) (drill 0.3) (layers "F.Cu" "B.Cu") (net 2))
 (via (at 124.44 83.23) (size 0.4) (drill 0.3) (layers "F.Cu" "B.Cu") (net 2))
 (via (at 125.25 83.23) (size 0.4) (drill 0.3) (layers "F.Cu" "B.Cu") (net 2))
 (via (at 127.85 83.23) (size 0.4) (drill 0.3) (layers "F.Cu" "B.Cu") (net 2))
 (via (at 127.1 83.23) (size 0.4) (drill 0.3) (layers "F.Cu" "B.Cu") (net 2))
 (via (at 125.32 79.809999) (size 0.4) (drill 0.3) (layers "F.Cu" "B.Cu") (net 2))
 (via (at 124.57 79.81) (size 0.4) (drill 0.3) (layers "F.Cu" "B.Cu") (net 2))
 (via (at 124.18 76.87) (size 0.4) (drill 0.3) (layers "F.Cu" "B.Cu") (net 2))
 (via (at 124.93 76.869999) (size 0.4) (drill 0.3) (layers "F.Cu" "B.Cu") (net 2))
 (via (at 124.93 76.099999) (size 0.4) (drill 0.3) (layers "F.Cu" "B.Cu") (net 2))
 (via (at 124.18 76.1) (size 0.4) (drill 0.3) (layers "F.Cu" "B.Cu") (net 2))
 (via (at 126.51 76.869999) (size 0.4) (drill 0.3) (layers "F.Cu" "B.Cu") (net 2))
 (via (at 125.76 76.1) (size 0.4) (drill 0.3) (layers "F.Cu" "B.Cu") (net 2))
 (via (at 125.76 76.87) (size 0.4) (drill 0.3) (layers "F.Cu" "B.Cu") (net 2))
 (via (at 126.51 76.099999) (size 0.4) (drill 0.3) (layers "F.Cu" "B.Cu") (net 2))
 (via (at 132.32 80.139999) (size 0.4) (drill 0.3) (layers "F.Cu" "B.Cu") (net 2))
 (via (at 131.57 80.91) (size 0.4) (drill 0.3) (layers "F.Cu" "B.Cu") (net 2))
 (via (at 132.32 80.909999) (size 0.4) (drill 0.3) (layers "F.Cu" "B.Cu") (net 2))
 (via (at 131.57 80.14) (size 0.4) (drill 0.3) (layers "F.Cu" "B.Cu") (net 2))
 (via (at 136.07 82.66) (size 0.4) (drill 0.3) (layers "F.Cu" "B.Cu") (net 2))
 (via (at 136.07 81.92) (size 0.4) (drill 0.3) (layers "F.Cu" "B.Cu") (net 2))
 (segment (start 139.52 82.06) (end 139.52 80.45) (width 0.5) (layer "F.Cu") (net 14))
 (segment (start 139.98 82.06) (end 139.98 80.45) (width 0.5) (layer "F.Cu") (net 14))
 (segment (start 140.47 80.515) (end 140.47 81.875) (width 0.5) (layer "F.Cu") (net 14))
 (segment (start 140.58001 82.30001) (end 140.805 82.525) (width 0.5) (layer "F.Cu") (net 14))
 (segment (start 140.805 80.515) (end 140.805 81.875) (width 0.5) (layer "F.Cu") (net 14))
 (segment (start 140.805 80.426458) (end 140.58001 80.201468) (width 0.5) (layer "F.Cu") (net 14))
 (segment (start 139.05 82.05) (end 139.05 80.44) (width 0.5) (layer "F.Cu") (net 14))
 (segment (start 140.805 80.515) (end 140.804999 78.565) (width 0.5) (layer "F.Cu") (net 14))
 (segment (start 140.805 80.515) (end 140.805 80.426458) (width 0.5) (layer "F.Cu") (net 14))
 (segment (start 140.58001 80.201468) (end 140.58001 82.30001) (width 0.5) (layer "F.Cu") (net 14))
 (segment (start 140.805 83.825) (end 140.805 81.875) (width 0.5) (layer "F.Cu") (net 14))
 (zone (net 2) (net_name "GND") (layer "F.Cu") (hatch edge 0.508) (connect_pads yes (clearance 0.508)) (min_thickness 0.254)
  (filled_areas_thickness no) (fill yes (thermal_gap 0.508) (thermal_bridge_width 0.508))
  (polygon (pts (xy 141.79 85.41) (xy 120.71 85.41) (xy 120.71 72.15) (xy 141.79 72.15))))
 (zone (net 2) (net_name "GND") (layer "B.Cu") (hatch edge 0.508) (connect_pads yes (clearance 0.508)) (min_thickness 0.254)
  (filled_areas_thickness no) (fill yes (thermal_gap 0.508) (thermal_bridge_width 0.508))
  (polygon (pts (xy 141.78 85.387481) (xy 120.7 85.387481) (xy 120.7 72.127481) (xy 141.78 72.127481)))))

